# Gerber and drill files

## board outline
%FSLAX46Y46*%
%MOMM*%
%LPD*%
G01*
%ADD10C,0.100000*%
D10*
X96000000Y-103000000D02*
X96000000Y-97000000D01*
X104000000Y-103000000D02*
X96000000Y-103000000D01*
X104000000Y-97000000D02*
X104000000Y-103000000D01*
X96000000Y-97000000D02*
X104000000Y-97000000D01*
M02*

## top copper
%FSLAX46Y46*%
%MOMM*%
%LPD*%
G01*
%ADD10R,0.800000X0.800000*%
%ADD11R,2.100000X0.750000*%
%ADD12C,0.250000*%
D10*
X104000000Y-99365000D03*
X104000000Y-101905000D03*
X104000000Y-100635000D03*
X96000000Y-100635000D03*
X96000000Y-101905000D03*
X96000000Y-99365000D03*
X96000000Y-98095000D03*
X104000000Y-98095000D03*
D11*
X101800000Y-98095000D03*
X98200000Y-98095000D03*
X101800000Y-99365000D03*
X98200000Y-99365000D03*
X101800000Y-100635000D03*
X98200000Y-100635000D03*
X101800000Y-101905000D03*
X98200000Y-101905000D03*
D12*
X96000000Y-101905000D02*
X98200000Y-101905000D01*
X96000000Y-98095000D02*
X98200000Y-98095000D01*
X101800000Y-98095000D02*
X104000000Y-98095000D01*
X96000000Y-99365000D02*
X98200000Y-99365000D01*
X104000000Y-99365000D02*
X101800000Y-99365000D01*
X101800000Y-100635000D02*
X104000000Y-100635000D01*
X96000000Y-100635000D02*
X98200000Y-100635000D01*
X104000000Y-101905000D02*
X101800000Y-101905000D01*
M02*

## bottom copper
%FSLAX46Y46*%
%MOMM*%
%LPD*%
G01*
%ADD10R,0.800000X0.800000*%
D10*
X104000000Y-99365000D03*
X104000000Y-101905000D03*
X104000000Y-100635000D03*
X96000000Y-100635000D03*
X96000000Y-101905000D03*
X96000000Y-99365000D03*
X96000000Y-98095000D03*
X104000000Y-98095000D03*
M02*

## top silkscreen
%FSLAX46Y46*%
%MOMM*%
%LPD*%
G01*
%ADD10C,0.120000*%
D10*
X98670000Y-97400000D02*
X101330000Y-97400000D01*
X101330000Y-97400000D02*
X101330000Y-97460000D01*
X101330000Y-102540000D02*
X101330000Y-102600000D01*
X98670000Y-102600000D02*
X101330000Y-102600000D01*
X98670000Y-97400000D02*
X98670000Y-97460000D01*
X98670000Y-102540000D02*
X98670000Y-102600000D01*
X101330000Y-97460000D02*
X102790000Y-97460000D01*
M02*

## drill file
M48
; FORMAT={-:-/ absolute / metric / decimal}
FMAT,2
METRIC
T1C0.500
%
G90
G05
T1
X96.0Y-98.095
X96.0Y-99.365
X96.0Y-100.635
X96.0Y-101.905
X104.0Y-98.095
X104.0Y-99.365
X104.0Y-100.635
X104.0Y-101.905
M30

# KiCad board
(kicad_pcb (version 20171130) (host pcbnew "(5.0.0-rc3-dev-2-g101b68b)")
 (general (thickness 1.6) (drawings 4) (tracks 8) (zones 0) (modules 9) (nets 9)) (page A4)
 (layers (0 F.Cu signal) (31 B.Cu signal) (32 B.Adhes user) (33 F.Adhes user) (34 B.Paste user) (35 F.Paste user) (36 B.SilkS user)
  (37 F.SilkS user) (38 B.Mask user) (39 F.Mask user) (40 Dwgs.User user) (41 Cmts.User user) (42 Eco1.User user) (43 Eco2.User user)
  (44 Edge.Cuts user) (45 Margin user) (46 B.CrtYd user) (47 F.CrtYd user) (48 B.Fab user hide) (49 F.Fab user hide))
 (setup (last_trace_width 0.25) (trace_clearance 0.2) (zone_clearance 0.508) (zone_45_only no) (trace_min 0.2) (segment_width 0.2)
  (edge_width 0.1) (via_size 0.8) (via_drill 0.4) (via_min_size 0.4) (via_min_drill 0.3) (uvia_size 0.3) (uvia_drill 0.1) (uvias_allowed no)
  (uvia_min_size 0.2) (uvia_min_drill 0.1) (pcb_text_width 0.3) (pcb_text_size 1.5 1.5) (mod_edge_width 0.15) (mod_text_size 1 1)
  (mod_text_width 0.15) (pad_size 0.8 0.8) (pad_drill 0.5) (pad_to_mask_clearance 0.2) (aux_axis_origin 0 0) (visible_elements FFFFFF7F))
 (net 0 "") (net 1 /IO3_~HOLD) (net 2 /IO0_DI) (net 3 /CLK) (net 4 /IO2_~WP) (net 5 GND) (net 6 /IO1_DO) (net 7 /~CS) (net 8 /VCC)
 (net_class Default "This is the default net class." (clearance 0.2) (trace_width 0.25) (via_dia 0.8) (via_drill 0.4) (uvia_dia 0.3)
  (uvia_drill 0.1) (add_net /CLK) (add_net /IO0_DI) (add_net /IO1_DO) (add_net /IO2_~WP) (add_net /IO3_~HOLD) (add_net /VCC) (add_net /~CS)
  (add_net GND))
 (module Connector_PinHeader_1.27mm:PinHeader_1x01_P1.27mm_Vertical (layer F.Cu) (at 104 99.365)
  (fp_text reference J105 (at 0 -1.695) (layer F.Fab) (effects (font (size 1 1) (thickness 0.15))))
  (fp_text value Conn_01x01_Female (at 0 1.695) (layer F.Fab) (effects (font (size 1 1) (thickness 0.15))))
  (pad 1 thru_hole rect (at 0 0) (size 0.8 0.8) (drill 0.5) (layers *.Cu *.Mask) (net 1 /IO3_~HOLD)))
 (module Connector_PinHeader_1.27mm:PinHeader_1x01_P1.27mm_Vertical (layer F.Cu) (at 104 101.905)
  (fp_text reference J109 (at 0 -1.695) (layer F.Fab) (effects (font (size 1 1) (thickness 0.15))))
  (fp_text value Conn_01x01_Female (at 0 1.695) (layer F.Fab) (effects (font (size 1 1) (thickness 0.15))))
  (pad 1 thru_hole rect (at 0 0) (size 0.8 0.8) (drill 0.5) (layers *.Cu *.Mask) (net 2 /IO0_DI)))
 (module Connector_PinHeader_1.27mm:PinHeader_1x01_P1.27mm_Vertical (layer F.Cu) (at 104 100.635)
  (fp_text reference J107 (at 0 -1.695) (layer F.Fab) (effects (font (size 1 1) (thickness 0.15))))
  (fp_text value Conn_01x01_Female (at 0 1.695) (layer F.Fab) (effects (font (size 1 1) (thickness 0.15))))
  (pad 1 thru_hole rect (at 0 0) (size 0.8 0.8) (drill 0.5) (layers *.Cu *.Mask) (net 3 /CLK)))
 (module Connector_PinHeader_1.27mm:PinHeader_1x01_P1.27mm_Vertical (layer F.Cu) (at 96 100.635)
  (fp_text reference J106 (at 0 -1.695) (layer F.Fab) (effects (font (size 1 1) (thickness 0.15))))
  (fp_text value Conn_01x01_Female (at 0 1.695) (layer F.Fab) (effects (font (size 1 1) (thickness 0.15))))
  (pad 1 thru_hole rect (at 0 0) (size 0.8 0.8) (drill 0.5) (layers *.Cu *.Mask) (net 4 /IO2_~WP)))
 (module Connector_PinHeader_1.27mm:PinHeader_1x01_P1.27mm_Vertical (layer F.Cu) (at 96 101.905)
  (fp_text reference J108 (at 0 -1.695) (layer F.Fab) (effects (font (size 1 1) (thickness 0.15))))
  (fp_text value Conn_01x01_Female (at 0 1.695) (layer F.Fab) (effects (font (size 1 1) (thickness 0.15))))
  (pad 1 thru_hole rect (at 0 0) (size 0.8 0.8) (drill 0.5) (layers *.Cu *.Mask) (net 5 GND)))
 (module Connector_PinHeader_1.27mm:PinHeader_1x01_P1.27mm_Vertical (layer F.Cu) (at 96 99.365)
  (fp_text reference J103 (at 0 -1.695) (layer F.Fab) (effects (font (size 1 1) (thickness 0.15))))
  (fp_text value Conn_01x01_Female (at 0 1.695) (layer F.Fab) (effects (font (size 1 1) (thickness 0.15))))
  (pad 1 thru_hole rect (at 0 0) (size 0.8 0.8) (drill 0.5) (layers *.Cu *.Mask) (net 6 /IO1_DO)))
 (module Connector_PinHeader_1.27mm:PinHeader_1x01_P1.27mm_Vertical (layer F.Cu) (at 96 98.095)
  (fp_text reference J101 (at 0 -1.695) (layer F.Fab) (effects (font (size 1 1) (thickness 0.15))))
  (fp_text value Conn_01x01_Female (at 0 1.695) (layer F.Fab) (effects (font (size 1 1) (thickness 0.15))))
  (pad 1 thru_hole rect (at 0 0) (size 0.8 0.8) (drill 0.5) (layers *.Cu *.Mask) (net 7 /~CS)))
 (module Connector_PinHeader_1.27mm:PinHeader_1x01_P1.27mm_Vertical (layer F.Cu) (at 104 98.095)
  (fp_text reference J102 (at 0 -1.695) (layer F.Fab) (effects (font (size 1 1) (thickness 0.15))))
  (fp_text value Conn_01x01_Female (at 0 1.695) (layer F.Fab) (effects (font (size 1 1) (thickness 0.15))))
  (pad 1 thru_hole rect (at 0 0) (size 0.8 0.8) (drill 0.5) (layers *.Cu *.Mask) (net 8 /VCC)))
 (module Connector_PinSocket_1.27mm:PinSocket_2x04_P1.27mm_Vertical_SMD (layer F.Cu) (at 100 100)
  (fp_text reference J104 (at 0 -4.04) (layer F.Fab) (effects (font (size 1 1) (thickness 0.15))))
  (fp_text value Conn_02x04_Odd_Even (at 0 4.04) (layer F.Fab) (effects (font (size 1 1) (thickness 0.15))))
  (fp_line (start -1.33 -2.6) (end 1.33 -2.6) (layer F.SilkS) (width 0.12))
  (fp_line (start 1.33 -2.6) (end 1.33 -2.54) (layer F.SilkS) (width 0.12))
  (fp_line (start 1.33 2.54) (end 1.33 2.6) (layer F.SilkS) (width 0.12))
  (fp_line (start -1.33 2.6) (end 1.33 2.6) (layer F.SilkS) (width 0.12))
  (fp_line (start -1.33 -2.6) (end -1.33 -2.54) (layer F.SilkS) (width 0.12))
  (fp_line (start -1.33 2.54) (end -1.33 2.6) (layer F.SilkS) (width 0.12))
  (fp_line (start 1.33 -2.54) (end 2.79 -2.54) (layer F.SilkS) (width 0.12))
  (pad 1 smd rect (at 1.8 -1.905) (size 2.1 0.75) (layers F.Cu F.Paste F.Mask) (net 8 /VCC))
  (pad 2 smd rect (at -1.8 -1.905) (size 2.1 0.75) (layers F.Cu F.Paste F.Mask) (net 7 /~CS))
  (pad 3 smd rect (at 1.8 -0.635) (size 2.1 0.75) (layers F.Cu F.Paste F.Mask) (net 1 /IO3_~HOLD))
  (pad 4 smd rect (at -1.8 -0.635) (size 2.1 0.75) (layers F.Cu F.Paste F.Mask) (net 6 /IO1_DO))
  (pad 5 smd rect (at 1.8 0.635) (size 2.1 0.75) (layers F.Cu F.Paste F.Mask) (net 3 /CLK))
  (pad 6 smd rect (at -1.8 0.635) (size 2.1 0.75) (layers F.Cu F.Paste F.Mask) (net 4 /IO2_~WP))
  (pad 7 smd rect (at 1.8 1.905) (size 2.1 0.75) (layers F.Cu F.Paste F.Mask) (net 2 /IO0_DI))
  (pad 8 smd rect (at -1.8 1.905) (size 2.1 0.75) (layers F.Cu F.Paste F.Mask) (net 5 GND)))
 (gr_line (start 96 103) (end 96 97) (layer Edge.Cuts) (width 0.1))
 (gr_line (start 104 103) (end 96 103) (layer Edge.Cuts) (width 0.1))
 (gr_line (start 104 97) (end 104 103) (layer Edge.Cuts) (width 0.1))
 (gr_line (start 96 97) (end 104 97) (layer Edge.Cuts) (width 0.1))
 (segment (start 96 101.905) (end 98.2 101.905) (width 0.25) (layer F.Cu) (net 5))
 (segment (start 96 98.095) (end 98.2 98.095) (width 0.25) (layer F.Cu) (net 7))
 (segment (start 101.8 98.095) (end 104 98.095) (width 0.25) (layer F.Cu) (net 8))
 (segment (start 96 99.365) (end 98.2 99.365) (width 0.25) (layer F.Cu) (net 6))
 (segment (start 104 99.365) (end 101.8 99.365) (width 0.25) (layer F.Cu) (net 1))
 (segment (start 101.8 100.635) (end 104 100.635) (width 0.25) (layer F.Cu) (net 3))
 (segment (start 96 100.635) (end 98.2 100.635) (width 0.25) (layer F.Cu) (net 4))
 (segment (start 104 101.905) (end 101.8 101.905) (width 0.25) (layer F.Cu) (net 2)))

